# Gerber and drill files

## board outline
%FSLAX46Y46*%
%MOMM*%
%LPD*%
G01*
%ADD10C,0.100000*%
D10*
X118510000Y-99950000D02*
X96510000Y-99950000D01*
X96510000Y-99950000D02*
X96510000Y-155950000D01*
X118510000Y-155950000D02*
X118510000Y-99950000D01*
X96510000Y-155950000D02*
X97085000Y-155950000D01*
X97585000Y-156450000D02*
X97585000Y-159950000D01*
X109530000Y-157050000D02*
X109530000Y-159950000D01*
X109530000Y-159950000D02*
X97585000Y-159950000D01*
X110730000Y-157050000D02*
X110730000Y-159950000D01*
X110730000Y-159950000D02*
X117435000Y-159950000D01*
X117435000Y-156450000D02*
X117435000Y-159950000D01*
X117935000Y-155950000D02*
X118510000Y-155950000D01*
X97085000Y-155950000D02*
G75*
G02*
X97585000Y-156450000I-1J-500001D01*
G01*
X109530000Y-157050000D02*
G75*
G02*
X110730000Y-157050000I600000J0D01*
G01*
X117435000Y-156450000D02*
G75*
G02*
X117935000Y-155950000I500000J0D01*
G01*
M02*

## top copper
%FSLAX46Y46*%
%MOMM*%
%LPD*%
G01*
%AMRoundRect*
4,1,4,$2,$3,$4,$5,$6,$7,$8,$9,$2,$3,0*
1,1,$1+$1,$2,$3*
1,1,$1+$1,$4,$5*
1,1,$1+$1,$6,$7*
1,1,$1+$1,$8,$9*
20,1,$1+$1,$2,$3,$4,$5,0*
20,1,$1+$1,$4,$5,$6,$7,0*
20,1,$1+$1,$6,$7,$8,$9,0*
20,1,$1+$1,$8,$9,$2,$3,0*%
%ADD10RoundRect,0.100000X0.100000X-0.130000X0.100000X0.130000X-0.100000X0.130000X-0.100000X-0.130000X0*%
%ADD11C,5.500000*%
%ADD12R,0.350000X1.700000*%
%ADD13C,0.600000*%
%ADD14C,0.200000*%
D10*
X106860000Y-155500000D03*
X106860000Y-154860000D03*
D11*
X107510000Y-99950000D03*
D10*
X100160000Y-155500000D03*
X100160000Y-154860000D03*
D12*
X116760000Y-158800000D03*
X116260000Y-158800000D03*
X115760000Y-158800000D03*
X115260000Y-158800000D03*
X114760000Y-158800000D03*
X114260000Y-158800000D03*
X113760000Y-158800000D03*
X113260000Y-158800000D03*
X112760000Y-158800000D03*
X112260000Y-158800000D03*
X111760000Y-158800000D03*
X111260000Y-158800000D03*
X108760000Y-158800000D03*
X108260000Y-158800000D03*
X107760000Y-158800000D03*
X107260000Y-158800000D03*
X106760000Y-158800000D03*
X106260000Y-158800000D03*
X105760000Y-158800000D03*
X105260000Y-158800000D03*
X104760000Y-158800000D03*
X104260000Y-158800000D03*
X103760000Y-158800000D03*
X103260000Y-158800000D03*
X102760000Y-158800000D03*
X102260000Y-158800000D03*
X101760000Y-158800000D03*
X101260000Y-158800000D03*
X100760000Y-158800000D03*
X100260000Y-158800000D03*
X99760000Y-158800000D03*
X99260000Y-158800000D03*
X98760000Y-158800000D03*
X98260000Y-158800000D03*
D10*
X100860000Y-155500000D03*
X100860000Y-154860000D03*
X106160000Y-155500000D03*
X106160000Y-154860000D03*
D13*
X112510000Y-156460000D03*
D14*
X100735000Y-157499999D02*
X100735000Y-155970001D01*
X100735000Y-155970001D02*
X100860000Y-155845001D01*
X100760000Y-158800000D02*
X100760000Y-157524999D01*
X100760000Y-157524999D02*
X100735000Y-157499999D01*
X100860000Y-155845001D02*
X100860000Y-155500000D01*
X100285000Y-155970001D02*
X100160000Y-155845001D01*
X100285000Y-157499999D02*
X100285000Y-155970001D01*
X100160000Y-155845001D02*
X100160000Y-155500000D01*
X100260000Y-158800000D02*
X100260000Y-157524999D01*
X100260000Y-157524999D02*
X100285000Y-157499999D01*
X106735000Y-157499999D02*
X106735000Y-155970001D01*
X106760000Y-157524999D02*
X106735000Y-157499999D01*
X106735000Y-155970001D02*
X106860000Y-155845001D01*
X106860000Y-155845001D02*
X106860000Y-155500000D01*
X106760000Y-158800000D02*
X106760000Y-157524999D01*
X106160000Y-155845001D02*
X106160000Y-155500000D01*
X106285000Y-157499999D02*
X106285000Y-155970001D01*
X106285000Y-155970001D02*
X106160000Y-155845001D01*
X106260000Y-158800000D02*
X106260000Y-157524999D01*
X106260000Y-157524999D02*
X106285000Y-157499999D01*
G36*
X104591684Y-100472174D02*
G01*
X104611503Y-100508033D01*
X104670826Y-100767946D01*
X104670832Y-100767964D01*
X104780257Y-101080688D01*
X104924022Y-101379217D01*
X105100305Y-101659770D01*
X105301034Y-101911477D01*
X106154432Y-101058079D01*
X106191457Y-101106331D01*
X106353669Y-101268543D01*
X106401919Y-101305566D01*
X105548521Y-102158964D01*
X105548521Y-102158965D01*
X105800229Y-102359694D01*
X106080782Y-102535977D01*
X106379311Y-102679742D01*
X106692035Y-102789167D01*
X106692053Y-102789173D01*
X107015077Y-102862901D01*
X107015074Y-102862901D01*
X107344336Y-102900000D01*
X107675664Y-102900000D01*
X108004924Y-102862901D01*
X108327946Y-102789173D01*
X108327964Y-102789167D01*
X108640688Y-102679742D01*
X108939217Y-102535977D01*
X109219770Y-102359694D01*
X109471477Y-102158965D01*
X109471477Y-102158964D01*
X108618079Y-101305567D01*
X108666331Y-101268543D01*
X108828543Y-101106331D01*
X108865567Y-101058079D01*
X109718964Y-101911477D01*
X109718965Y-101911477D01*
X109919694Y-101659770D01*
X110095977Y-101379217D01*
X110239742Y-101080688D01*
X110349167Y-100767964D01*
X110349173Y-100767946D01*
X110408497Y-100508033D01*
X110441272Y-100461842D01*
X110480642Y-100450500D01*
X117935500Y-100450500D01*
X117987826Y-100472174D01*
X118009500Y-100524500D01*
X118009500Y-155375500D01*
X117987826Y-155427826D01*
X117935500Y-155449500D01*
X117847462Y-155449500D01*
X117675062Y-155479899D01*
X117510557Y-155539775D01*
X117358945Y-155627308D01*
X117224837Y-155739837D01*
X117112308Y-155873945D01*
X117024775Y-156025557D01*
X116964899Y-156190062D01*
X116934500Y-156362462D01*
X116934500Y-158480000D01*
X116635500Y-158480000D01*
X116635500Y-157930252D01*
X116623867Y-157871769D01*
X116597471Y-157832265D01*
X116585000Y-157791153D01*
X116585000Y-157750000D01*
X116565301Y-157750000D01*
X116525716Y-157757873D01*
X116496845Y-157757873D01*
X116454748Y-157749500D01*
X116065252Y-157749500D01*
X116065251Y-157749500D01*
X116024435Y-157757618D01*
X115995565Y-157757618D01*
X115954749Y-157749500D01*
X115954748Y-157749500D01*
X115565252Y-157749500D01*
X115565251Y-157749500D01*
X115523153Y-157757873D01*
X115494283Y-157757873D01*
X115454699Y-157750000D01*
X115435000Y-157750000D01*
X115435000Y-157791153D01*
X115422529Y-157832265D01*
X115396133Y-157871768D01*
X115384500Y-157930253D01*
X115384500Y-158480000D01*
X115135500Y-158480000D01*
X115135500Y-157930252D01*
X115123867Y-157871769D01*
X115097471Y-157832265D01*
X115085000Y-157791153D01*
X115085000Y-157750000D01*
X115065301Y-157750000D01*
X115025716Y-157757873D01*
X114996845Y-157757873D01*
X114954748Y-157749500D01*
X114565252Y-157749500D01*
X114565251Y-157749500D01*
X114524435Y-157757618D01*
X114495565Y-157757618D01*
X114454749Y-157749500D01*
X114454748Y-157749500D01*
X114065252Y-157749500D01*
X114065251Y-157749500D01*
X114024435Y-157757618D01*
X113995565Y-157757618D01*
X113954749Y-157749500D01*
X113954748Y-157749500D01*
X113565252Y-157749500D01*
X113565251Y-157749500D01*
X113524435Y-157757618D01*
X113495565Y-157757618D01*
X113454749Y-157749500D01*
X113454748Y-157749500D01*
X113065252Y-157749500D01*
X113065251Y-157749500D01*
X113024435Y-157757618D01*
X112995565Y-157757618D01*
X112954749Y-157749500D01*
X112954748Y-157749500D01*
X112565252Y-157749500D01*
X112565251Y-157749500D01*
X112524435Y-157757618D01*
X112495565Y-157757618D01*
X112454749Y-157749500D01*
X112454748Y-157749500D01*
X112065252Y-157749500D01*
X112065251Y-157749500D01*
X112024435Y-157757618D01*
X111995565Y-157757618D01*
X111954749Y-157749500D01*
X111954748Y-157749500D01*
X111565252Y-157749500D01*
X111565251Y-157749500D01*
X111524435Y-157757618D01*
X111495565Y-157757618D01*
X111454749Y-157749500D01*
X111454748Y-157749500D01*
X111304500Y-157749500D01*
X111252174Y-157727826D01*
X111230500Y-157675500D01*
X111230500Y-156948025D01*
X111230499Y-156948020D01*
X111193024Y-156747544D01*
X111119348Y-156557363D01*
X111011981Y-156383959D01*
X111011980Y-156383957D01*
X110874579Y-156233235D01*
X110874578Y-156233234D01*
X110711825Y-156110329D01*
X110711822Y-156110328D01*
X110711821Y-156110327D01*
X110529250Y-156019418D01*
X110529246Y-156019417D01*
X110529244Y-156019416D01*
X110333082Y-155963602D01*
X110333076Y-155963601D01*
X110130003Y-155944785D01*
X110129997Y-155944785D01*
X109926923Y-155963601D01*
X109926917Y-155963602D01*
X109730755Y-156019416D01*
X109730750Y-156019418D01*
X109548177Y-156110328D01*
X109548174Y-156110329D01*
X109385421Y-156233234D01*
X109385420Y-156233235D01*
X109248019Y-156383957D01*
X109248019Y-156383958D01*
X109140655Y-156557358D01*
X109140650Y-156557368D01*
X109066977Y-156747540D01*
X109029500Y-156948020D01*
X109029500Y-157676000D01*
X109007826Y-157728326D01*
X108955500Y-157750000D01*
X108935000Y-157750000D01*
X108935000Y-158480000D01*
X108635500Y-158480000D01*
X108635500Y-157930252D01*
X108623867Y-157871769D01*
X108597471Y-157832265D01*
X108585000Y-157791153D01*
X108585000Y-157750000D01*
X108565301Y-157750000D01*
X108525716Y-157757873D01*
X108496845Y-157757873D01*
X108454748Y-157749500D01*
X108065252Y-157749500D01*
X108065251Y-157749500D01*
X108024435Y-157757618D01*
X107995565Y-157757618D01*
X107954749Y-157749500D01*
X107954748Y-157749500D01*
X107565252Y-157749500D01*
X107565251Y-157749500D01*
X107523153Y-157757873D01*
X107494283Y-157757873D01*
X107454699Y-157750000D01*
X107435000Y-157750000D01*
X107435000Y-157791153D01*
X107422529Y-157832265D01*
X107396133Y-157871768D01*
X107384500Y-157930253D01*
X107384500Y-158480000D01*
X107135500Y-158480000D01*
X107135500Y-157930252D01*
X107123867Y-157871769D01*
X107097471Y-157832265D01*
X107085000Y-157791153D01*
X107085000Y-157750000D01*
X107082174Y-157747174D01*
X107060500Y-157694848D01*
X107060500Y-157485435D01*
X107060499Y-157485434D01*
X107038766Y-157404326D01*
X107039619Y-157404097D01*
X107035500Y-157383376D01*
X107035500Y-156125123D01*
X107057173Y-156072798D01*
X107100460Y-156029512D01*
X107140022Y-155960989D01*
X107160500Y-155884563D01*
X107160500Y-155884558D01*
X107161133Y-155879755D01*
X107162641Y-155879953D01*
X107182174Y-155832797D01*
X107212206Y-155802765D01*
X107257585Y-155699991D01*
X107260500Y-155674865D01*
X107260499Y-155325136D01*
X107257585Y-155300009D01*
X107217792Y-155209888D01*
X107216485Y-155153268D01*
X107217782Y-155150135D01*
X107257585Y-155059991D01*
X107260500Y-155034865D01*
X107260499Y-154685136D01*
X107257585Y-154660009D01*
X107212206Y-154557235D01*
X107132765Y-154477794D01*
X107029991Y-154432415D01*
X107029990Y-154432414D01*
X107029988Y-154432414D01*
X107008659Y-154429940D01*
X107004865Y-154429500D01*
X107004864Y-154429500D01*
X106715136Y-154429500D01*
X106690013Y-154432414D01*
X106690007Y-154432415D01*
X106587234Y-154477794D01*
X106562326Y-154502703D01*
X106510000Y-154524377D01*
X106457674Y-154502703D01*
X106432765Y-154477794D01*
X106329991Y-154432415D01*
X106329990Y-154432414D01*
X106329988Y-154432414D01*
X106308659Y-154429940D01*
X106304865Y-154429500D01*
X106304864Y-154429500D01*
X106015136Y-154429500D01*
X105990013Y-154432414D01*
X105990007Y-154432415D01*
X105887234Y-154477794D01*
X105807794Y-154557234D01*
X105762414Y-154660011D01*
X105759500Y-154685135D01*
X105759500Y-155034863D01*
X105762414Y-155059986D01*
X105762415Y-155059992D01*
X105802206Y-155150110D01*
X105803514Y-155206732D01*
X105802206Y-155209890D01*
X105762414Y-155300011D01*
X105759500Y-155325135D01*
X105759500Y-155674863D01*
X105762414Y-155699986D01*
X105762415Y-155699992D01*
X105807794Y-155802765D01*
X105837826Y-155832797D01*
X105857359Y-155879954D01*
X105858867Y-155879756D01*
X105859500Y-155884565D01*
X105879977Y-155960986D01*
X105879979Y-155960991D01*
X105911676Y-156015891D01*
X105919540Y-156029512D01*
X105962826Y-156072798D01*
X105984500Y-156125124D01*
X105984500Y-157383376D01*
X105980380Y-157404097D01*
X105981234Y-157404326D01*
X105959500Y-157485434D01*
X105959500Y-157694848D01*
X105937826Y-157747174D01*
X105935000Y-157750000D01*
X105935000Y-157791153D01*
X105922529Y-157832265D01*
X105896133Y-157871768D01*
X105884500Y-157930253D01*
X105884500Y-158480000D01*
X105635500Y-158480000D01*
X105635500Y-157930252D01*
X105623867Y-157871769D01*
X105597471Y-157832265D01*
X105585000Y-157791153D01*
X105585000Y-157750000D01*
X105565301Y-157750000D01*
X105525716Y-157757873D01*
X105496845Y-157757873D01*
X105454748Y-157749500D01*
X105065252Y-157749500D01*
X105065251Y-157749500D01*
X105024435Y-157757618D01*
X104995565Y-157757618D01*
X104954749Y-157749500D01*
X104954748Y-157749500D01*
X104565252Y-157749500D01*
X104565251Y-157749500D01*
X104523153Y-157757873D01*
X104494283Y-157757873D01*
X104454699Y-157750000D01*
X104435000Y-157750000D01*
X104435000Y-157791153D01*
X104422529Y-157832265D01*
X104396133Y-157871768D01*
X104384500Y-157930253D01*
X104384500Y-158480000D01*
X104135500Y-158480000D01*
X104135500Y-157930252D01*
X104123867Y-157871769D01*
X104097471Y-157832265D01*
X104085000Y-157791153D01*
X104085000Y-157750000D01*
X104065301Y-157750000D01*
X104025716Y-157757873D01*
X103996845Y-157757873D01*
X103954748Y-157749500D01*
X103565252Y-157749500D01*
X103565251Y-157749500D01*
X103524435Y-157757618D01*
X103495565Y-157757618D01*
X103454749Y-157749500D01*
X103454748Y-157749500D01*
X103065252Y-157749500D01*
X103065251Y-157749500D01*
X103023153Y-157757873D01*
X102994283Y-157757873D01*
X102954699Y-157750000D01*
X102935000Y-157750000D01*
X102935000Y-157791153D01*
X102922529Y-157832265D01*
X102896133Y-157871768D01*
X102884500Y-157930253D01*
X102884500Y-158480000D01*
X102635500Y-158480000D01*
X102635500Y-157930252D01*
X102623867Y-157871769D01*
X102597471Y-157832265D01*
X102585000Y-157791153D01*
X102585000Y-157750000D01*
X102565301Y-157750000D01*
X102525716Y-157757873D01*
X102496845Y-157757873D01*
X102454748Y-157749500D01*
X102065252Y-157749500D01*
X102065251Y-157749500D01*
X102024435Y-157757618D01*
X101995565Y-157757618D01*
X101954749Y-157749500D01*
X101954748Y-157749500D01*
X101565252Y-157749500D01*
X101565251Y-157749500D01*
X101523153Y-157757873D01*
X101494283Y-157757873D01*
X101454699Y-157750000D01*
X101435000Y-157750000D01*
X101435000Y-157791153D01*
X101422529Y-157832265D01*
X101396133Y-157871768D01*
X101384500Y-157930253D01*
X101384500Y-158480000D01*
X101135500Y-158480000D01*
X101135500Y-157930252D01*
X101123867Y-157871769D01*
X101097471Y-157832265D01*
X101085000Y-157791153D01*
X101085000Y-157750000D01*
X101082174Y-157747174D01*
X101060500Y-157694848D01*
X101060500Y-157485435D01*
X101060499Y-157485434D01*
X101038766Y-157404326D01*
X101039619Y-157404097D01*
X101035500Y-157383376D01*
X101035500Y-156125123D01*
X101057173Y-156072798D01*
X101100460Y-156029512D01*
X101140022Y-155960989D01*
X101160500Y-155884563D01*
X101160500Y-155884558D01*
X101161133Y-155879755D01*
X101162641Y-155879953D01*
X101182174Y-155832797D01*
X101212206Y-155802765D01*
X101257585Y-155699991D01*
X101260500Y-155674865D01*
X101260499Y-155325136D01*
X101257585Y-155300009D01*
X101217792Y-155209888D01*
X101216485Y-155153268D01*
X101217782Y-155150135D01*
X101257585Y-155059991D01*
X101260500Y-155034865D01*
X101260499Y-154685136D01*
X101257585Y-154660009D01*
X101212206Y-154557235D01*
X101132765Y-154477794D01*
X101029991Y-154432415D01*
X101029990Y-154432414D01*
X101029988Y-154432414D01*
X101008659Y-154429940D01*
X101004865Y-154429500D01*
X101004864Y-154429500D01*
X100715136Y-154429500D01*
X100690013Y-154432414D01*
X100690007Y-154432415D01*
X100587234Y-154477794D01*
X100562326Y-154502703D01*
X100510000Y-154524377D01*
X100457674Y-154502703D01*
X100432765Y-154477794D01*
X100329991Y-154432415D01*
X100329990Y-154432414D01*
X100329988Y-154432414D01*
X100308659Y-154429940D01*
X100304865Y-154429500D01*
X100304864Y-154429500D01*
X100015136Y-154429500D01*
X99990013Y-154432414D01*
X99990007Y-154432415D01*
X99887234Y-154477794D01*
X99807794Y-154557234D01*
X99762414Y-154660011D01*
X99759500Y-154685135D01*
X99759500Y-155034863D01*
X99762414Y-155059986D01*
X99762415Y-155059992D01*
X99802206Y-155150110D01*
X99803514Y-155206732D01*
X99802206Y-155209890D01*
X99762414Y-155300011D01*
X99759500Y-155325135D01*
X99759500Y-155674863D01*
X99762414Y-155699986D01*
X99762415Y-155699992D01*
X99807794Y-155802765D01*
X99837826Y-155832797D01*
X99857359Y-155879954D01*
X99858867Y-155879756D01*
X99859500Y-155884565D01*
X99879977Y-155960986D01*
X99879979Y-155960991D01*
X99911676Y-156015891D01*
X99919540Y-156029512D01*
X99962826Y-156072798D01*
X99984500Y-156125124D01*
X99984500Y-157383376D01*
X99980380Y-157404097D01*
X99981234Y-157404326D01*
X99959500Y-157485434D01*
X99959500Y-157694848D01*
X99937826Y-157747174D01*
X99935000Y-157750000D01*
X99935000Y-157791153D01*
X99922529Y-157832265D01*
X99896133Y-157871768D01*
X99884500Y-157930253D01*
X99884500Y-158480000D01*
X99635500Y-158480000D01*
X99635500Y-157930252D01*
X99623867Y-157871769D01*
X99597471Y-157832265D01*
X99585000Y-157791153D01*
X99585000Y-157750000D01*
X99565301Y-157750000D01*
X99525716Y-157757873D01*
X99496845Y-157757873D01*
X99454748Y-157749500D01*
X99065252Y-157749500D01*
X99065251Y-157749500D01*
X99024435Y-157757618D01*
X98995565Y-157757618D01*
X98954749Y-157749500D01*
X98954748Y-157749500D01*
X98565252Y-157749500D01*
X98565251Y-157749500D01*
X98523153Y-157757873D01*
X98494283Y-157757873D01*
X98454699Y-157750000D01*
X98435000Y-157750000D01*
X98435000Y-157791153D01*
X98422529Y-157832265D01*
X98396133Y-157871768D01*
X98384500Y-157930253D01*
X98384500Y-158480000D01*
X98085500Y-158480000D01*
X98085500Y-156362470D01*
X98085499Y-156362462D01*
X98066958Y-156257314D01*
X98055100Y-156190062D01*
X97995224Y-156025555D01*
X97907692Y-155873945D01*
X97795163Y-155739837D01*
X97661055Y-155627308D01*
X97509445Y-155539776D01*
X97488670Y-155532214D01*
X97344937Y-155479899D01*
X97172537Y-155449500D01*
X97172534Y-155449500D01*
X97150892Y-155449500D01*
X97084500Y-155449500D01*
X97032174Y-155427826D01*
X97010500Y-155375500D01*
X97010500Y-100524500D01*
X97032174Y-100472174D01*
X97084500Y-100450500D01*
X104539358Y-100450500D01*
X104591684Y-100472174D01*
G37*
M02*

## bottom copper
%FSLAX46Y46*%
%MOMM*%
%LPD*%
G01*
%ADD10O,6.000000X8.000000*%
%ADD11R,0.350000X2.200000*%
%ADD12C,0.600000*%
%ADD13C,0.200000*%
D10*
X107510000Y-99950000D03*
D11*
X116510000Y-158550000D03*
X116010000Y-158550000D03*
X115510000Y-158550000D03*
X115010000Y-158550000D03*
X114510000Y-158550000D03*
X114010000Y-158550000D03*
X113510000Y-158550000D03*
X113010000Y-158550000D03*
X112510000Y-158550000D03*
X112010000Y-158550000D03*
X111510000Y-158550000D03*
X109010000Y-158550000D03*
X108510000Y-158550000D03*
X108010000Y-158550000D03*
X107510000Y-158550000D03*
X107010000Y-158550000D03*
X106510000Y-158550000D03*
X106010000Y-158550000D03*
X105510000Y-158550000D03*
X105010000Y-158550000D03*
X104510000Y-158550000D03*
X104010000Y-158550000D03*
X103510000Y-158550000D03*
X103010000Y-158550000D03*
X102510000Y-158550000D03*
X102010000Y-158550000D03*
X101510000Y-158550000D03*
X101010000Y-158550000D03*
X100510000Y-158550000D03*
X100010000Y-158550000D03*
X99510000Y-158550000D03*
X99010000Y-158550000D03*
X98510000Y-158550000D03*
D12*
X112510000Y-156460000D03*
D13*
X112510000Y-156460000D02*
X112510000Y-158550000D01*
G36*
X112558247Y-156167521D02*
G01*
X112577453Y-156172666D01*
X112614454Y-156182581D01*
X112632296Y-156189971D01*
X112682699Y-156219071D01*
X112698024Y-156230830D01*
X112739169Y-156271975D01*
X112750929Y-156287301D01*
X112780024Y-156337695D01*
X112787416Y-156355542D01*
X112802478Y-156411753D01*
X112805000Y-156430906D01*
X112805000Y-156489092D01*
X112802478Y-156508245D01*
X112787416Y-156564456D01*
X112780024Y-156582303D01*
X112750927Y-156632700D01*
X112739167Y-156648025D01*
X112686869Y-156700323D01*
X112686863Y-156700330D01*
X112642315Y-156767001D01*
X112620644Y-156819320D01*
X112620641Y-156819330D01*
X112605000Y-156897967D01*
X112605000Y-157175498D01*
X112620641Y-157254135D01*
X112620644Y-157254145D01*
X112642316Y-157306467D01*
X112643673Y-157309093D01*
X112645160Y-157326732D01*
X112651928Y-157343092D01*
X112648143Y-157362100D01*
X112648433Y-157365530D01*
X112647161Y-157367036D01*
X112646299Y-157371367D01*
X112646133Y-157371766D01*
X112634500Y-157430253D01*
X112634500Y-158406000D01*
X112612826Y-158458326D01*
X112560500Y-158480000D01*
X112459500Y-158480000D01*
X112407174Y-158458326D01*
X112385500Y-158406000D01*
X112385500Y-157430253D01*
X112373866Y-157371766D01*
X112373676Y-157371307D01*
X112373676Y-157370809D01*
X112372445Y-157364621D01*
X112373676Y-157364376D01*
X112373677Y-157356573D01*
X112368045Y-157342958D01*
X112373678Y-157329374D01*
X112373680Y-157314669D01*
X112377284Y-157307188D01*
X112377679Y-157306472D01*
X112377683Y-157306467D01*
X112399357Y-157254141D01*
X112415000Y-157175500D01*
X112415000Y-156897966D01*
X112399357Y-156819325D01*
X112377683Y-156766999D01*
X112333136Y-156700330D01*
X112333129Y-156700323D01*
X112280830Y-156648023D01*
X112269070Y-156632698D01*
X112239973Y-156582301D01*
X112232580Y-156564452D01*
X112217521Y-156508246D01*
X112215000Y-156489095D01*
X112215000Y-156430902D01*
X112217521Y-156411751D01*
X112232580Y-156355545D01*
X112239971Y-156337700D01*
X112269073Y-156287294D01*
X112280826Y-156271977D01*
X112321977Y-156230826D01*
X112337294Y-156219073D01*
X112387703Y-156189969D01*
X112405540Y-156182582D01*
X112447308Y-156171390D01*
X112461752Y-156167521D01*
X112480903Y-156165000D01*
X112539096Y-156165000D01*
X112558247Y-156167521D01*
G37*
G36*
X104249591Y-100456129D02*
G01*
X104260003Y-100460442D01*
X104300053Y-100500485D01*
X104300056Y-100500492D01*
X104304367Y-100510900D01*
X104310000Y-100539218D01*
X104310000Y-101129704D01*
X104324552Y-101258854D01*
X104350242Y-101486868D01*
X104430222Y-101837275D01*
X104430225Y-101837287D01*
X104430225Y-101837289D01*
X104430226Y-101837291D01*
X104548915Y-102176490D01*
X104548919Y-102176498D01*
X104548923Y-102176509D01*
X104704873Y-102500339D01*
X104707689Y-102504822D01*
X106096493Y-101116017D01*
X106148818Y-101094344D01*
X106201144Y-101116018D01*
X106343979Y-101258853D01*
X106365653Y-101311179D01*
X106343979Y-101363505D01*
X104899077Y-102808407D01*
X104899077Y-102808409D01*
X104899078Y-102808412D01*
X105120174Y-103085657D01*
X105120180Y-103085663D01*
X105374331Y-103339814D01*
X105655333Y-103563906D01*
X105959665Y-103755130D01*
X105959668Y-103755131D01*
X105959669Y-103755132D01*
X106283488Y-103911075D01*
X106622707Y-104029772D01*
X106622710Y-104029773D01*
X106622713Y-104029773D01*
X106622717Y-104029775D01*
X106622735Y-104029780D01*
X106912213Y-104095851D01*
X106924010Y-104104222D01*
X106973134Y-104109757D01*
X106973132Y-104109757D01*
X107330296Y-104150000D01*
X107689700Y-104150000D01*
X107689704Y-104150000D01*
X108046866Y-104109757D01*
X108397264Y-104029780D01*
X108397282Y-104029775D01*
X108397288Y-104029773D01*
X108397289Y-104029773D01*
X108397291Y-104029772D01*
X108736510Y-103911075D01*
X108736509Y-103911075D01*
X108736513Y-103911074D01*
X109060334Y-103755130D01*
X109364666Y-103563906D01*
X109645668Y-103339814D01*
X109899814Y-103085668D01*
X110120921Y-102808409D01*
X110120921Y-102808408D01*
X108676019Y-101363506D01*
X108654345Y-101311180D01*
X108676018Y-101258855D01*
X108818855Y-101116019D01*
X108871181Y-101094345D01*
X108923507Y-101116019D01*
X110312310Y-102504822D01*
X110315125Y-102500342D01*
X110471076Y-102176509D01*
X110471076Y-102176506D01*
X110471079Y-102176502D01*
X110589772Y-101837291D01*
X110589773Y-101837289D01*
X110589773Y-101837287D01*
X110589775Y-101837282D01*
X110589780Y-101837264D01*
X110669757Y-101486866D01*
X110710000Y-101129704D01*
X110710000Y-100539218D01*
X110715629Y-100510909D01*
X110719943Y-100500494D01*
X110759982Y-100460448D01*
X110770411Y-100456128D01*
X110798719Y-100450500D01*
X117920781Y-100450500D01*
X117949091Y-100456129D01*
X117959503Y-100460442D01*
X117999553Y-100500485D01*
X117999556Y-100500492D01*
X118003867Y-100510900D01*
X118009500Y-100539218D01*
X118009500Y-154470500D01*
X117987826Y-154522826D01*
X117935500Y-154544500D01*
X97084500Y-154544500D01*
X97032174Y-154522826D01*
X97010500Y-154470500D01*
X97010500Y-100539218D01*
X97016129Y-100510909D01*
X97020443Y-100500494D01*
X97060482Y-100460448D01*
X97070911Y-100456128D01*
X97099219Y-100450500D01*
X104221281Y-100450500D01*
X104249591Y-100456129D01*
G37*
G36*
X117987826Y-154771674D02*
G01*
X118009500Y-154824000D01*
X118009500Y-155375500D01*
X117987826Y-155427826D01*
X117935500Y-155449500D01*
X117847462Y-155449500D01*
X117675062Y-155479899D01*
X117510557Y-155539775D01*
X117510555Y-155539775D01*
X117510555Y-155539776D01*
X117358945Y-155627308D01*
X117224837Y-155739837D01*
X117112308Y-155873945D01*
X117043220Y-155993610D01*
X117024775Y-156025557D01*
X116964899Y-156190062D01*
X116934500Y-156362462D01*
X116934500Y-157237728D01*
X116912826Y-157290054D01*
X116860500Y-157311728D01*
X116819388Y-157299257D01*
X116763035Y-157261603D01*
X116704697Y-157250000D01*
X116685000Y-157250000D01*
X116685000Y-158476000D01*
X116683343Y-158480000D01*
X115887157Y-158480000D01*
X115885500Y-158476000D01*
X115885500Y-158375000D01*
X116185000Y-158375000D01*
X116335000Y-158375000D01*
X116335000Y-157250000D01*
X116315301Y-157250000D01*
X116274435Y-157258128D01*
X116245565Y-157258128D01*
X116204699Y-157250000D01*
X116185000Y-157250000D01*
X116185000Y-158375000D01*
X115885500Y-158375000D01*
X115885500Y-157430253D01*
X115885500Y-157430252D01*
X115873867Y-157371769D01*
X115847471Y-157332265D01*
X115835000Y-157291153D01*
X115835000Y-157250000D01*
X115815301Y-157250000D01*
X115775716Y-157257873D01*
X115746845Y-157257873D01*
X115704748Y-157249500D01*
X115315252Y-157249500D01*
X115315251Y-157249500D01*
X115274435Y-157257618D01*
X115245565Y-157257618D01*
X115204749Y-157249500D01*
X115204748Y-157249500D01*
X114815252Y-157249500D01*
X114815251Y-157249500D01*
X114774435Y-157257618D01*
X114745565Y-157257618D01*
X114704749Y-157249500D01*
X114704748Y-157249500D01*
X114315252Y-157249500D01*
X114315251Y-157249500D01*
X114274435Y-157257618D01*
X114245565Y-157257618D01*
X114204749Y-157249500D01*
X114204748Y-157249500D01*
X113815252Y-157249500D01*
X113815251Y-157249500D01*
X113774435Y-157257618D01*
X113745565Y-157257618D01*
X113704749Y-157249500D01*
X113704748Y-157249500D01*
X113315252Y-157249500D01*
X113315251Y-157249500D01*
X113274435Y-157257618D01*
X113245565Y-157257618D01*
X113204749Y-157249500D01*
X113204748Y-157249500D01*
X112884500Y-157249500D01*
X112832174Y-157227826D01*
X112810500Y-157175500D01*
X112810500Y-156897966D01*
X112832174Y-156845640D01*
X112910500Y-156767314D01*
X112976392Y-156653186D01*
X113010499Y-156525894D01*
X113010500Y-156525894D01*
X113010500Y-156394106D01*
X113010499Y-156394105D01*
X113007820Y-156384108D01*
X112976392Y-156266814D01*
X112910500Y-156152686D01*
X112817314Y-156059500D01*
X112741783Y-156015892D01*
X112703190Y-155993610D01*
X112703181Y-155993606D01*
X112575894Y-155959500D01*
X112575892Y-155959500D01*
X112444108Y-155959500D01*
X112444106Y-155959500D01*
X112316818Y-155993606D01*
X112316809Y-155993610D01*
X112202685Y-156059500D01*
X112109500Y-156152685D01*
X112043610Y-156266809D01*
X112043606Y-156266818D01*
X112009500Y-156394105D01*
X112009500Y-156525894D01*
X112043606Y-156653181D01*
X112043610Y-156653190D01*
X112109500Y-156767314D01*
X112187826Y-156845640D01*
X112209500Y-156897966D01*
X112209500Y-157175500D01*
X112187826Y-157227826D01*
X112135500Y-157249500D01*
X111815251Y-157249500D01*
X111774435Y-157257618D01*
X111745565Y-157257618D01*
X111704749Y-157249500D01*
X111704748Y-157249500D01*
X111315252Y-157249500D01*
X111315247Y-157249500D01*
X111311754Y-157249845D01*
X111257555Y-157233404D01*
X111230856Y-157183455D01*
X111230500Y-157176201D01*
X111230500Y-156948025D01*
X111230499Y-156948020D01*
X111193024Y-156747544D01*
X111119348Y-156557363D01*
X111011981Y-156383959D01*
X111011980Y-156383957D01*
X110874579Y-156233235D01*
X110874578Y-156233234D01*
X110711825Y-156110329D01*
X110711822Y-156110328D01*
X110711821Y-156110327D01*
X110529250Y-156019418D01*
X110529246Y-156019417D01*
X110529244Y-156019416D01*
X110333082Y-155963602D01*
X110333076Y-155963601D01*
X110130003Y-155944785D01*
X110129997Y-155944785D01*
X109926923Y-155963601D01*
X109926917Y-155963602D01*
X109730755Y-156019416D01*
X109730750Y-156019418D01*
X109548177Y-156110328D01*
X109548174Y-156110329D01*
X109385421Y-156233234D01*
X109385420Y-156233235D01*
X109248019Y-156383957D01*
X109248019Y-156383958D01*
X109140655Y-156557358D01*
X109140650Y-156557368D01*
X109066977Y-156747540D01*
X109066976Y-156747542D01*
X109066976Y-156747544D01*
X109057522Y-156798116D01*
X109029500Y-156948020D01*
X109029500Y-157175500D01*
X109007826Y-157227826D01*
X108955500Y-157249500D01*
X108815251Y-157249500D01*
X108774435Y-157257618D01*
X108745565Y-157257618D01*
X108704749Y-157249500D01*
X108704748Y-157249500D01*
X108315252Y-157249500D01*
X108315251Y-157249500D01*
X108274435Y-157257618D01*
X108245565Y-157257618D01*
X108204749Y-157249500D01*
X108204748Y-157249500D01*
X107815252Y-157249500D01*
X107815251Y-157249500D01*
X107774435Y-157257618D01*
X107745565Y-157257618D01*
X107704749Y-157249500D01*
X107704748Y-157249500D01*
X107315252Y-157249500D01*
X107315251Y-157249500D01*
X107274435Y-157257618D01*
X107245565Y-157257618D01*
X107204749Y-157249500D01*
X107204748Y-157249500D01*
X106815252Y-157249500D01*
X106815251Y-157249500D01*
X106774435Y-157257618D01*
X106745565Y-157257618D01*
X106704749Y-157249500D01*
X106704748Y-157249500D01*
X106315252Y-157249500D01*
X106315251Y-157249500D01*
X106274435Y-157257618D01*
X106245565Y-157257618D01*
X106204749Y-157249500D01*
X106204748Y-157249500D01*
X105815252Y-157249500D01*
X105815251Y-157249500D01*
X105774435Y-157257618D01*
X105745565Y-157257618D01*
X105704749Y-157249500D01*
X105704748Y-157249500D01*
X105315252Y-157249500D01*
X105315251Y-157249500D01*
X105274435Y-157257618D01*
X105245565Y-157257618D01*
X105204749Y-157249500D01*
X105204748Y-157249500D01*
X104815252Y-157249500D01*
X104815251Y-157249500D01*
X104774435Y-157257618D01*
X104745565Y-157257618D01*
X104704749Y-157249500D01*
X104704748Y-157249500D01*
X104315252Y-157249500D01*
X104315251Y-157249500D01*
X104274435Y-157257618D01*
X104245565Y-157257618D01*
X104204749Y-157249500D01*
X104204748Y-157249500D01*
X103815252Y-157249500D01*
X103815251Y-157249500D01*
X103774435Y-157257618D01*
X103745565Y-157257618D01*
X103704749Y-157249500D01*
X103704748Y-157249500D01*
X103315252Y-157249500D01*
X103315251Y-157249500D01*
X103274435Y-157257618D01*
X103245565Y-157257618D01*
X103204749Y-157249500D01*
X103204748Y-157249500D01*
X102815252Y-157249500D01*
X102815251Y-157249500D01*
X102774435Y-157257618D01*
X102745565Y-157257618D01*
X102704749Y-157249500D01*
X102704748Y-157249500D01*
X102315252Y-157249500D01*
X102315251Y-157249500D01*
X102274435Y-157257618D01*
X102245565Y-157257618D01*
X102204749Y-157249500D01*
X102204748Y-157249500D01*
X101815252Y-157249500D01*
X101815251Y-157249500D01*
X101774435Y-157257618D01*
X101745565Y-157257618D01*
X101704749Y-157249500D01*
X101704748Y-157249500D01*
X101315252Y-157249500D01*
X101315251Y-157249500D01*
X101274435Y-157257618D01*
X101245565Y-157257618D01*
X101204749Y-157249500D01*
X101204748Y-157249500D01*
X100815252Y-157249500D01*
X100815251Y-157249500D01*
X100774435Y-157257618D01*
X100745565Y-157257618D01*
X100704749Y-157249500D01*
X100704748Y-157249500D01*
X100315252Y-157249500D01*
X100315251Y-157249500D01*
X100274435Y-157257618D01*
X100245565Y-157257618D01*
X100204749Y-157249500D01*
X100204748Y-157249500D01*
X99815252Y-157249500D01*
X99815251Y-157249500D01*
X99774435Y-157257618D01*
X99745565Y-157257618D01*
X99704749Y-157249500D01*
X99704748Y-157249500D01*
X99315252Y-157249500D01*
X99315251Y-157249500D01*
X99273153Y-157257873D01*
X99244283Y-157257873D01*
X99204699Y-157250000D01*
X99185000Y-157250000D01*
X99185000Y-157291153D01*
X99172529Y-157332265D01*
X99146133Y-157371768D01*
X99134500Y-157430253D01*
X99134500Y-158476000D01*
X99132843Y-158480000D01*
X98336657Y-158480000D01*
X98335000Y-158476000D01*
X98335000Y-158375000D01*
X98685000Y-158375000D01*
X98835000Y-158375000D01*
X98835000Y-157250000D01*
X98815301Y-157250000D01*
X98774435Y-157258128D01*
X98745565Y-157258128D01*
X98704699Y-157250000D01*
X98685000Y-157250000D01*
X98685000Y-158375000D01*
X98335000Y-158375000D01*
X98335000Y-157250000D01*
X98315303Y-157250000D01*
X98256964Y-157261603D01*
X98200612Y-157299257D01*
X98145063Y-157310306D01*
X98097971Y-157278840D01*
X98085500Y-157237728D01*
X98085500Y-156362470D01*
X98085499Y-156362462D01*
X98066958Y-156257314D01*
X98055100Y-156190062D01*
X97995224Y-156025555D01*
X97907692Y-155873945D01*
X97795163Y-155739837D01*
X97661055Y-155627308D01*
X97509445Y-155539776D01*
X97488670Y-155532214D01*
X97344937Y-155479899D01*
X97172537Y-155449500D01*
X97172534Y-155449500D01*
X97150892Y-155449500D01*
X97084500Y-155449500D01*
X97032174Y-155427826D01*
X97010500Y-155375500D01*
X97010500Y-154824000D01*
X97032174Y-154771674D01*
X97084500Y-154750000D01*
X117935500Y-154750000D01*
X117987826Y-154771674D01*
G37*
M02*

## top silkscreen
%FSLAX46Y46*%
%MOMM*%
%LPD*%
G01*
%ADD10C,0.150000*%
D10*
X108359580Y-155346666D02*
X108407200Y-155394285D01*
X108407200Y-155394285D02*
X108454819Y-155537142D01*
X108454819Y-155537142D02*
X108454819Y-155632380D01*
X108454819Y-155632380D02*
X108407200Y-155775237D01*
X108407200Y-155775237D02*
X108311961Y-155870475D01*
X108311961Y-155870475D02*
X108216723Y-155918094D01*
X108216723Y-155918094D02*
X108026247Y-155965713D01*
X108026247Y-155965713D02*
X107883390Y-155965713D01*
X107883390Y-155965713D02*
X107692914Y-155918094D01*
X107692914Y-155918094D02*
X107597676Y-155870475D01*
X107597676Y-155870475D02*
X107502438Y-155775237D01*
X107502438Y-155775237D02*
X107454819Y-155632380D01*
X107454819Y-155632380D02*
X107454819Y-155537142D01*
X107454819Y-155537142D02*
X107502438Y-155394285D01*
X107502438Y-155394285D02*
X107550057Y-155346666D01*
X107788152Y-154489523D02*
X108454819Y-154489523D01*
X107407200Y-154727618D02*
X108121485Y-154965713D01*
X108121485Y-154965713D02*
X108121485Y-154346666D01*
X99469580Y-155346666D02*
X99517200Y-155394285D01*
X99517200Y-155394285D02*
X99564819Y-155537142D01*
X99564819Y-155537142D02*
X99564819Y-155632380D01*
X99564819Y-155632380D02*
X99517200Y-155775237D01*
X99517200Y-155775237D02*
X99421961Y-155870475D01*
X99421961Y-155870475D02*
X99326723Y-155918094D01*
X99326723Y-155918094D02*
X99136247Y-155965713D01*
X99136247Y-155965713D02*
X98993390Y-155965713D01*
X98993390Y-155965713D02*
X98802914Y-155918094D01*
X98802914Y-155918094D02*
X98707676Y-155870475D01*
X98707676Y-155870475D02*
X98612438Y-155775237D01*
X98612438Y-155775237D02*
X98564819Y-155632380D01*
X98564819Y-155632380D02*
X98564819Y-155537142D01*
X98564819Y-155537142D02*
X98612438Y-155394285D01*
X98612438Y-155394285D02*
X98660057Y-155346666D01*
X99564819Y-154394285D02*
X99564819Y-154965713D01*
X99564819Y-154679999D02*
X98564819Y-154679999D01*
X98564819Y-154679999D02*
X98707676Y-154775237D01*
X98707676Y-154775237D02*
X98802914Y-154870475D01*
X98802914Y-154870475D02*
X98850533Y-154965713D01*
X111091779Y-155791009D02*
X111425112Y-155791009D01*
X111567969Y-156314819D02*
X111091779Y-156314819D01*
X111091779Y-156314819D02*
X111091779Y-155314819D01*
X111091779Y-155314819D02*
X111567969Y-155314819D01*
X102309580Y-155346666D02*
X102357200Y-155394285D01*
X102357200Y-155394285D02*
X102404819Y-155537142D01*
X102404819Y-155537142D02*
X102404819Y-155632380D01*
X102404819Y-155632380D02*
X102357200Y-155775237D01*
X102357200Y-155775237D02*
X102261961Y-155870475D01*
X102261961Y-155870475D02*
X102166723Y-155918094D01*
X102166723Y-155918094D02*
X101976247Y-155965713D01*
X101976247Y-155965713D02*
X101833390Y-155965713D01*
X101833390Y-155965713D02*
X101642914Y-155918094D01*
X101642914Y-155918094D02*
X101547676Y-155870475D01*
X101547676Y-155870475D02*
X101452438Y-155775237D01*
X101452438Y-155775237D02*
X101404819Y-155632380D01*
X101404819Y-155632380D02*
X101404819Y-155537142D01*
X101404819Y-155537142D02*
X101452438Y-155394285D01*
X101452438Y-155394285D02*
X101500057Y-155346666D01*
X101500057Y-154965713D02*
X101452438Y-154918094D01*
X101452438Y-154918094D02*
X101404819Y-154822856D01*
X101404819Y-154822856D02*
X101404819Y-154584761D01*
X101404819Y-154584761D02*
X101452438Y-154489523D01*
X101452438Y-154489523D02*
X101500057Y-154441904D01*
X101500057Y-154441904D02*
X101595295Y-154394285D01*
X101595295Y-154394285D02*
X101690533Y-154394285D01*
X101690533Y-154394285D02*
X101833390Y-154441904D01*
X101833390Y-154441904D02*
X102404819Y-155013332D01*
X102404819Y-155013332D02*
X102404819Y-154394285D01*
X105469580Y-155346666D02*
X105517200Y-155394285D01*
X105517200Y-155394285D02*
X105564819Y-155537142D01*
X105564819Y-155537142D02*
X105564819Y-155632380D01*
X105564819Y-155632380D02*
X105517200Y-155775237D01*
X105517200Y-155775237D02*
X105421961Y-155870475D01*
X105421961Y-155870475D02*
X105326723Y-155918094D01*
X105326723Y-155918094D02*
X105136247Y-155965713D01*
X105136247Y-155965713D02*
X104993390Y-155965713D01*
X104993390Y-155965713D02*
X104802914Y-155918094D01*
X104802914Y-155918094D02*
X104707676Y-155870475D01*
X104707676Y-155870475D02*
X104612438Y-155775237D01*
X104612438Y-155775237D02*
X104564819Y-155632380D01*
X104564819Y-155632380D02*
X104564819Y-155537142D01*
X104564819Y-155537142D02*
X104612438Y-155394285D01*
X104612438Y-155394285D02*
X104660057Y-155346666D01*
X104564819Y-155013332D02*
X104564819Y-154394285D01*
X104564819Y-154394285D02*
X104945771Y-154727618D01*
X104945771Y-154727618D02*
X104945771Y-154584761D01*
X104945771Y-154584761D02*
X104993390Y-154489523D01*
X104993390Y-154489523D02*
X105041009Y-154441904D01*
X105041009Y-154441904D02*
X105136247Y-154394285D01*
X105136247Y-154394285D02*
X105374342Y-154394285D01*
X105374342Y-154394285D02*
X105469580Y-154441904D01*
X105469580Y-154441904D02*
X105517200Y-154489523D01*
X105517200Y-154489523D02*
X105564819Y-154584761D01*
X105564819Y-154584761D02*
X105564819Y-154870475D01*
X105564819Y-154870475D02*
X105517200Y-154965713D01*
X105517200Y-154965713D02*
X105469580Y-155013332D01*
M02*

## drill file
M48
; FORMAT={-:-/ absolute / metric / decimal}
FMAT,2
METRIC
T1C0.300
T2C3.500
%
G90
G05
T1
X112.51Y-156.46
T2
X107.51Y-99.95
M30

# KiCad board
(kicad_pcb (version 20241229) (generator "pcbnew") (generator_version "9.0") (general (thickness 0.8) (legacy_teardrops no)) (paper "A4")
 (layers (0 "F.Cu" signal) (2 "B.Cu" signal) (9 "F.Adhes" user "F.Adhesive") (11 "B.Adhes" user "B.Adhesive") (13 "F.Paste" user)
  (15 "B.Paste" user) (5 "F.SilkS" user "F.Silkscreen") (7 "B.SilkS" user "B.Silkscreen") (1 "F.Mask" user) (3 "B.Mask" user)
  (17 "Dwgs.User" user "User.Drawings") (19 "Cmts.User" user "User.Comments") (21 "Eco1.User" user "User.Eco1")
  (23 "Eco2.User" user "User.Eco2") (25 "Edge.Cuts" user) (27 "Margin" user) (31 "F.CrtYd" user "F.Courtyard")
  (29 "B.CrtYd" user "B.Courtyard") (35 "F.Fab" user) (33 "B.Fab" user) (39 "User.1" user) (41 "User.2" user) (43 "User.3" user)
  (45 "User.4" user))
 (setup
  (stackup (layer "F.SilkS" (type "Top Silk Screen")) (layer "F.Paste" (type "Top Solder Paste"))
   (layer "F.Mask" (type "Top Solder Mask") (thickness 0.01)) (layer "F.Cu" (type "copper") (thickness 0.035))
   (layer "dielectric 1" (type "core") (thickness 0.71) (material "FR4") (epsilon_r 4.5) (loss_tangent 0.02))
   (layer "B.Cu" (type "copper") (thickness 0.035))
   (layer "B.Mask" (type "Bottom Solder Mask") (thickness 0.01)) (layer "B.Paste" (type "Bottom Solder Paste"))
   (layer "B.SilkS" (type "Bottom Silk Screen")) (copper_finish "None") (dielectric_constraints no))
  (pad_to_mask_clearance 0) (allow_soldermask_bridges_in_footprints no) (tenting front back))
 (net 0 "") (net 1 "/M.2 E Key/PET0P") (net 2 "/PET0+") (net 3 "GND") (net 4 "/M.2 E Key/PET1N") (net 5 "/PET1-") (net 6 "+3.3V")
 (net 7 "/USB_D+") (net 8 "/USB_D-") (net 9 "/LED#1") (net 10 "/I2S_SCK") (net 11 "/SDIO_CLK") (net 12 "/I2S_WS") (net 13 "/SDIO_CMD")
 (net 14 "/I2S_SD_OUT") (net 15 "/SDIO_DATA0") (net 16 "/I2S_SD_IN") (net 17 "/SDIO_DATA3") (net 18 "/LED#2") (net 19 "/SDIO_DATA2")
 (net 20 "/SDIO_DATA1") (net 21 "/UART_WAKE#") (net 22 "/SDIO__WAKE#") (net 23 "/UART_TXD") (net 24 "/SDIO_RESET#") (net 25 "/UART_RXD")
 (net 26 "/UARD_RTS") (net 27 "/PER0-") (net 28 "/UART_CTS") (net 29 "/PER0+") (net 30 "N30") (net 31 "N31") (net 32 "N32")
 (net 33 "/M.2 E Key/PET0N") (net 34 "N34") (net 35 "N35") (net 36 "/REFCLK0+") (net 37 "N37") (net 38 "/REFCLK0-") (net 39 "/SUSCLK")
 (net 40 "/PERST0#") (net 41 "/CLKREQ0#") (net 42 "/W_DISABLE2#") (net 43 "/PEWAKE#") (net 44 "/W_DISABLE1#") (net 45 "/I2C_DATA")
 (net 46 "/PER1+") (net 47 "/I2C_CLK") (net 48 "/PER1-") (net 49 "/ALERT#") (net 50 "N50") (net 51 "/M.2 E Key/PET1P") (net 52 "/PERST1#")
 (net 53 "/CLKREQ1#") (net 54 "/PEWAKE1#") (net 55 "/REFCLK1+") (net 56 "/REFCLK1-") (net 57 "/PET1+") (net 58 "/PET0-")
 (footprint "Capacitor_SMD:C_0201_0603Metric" (layer "F.Cu") (at 106.86 155.18 90)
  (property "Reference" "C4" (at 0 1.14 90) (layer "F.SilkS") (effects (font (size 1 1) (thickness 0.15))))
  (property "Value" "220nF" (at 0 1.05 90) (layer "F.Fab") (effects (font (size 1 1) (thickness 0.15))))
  (pad "" smd roundrect (at -0.345 0 90) (size 0.318 0.36) (layers "F.Paste") (roundrect_rratio 0.25))
  (pad "" smd roundrect (at 0.345 0 90) (size 0.318 0.36) (layers "F.Paste") (roundrect_rratio 0.25))
  (pad "1" smd roundrect (at -0.32 0 90) (size 0.46 0.4) (layers "F.Cu" "F.Mask") (roundrect_rratio 0.25) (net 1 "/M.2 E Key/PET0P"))
  (pad "2" smd roundrect (at 0.32 0 90) (size 0.46 0.4) (layers "F.Cu" "F.Mask") (roundrect_rratio 0.25) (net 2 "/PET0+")))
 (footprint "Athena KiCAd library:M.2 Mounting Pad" (layer "F.Cu") (at 107.51 99.95)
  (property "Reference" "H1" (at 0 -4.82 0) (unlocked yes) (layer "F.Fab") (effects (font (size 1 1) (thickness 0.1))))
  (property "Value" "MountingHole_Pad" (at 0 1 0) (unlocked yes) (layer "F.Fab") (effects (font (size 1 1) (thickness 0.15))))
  (pad "1" thru_hole circle (at 0 0) (size 5.5 5.5) (drill 3.5) (layers "*.Cu" "*.Mask") (remove_unused_layers no) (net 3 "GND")
   (padstack (mode front_inner_back)
    (layer "Inner" (shape circle) (size 5.5 5.5) (zone_connect -1))
    (layer "B.Cu" (shape oval) (size 6 8) (thermal_bridge_angle 45) (zone_connect -1)))))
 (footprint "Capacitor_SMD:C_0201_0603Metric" (layer "F.Cu") (at 100.16 155.18 90)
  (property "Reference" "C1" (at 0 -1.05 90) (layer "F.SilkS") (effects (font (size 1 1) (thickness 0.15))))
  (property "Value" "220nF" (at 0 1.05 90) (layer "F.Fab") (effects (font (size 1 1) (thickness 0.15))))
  (pad "" smd roundrect (at -0.345 0 90) (size 0.318 0.36) (layers "F.Paste") (roundrect_rratio 0.25))
  (pad "" smd roundrect (at 0.345 0 90) (size 0.318 0.36) (layers "F.Paste") (roundrect_rratio 0.25))
  (pad "1" smd roundrect (at -0.32 0 90) (size 0.46 0.4) (layers "F.Cu" "F.Mask") (roundrect_rratio 0.25) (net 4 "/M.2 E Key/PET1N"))
  (pad "2" smd roundrect (at 0.32 0 90) (size 0.46 0.4) (layers "F.Cu" "F.Mask") (roundrect_rratio 0.25) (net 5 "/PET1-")))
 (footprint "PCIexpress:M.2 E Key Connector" (layer "F.Cu") (at 107.51 158.84)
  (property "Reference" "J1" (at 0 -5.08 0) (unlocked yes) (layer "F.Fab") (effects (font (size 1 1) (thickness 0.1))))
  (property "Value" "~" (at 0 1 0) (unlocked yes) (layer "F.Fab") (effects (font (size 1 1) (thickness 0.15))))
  (fp_line (start -11 -2.89) (end -10.425 -2.89) (stroke (width 0.1) (type default)) (layer "Edge.Cuts"))
  (fp_line (start -9.925 -2.39) (end -9.925 1.11) (stroke (width 0.1) (type default)) (layer "Edge.Cuts"))
  (fp_line (start 2.02 -1.79) (end 2.02 1.11) (stroke (width 0.1) (type default)) (layer "Edge.Cuts"))
  (fp_line (start 2.02 1.11) (end -9.925 1.11) (stroke (width 0.1) (type default)) (layer "Edge.Cuts"))
  (fp_line (start 3.22 -1.79) (end 3.22 1.11) (stroke (width 0.1) (type default)) (layer "Edge.Cuts"))
  (fp_line (start 3.22 1.11) (end 9.925 1.11) (stroke (width 0.1) (type default)) (layer "Edge.Cuts"))
  (fp_line (start 9.925 -2.39) (end 9.925 1.11) (stroke (width 0.1) (type default)) (layer "Edge.Cuts"))
  (fp_line (start 10.425 -2.89) (end 11 -2.89) (stroke (width 0.1) (type default)) (layer "Edge.Cuts"))
  (fp_arc (start -10.425 -2.89) (mid -10.071447 -2.743553) (end -9.925 -2.39) (stroke (width 0.1) (type default)) (layer "Edge.Cuts"))
  (fp_arc (start 2.02 -1.79) (mid 2.62 -2.39) (end 3.22 -1.79) (stroke (width 0.1) (type default)) (layer "Edge.Cuts"))
  (fp_arc (start 9.925 -2.39) (mid 10.071447 -2.743553) (end 10.425 -2.89) (stroke (width 0.1) (type default)) (layer "Edge.Cuts"))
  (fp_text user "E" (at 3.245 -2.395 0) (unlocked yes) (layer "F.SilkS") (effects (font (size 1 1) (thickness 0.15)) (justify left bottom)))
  (pad "1" smd rect (at 9.25 -0.04 180) (size 0.35 1.7) (layers "F.Cu") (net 3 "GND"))
  (pad "2" smd rect (at 9 -0.29 180) (size 0.35 2.2) (layers "B.Cu") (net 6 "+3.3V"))
  (pad "3" smd rect (at 8.75 -0.04 180) (size 0.35 1.7) (layers "F.Cu") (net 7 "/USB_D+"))
  (pad "4" smd rect (at 8.5 -0.29 180) (size 0.35 2.2) (layers "B.Cu") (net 6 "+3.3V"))
  (pad "5" smd rect (at 8.25 -0.04 180) (size 0.35 1.7) (layers "F.Cu") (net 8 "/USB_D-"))
  (pad "6" smd rect (at 8 -0.29 180) (size 0.35 2.2) (layers "B.Cu") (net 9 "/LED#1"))
  (pad "7" smd rect (at 7.75 -0.04 180) (size 0.35 1.7) (layers "F.Cu") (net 3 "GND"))
  (pad "8" smd rect (at 7.5 -0.29 180) (size 0.35 2.2) (layers "B.Cu") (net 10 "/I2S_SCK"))
  (pad "9" smd rect (at 7.25 -0.04 180) (size 0.35 1.7) (layers "F.Cu") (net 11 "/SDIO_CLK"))
  (pad "10" smd rect (at 7 -0.29 180) (size 0.35 2.2) (layers "B.Cu") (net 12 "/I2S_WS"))
  (pad "11" smd rect (at 6.75 -0.04 180) (size 0.35 1.7) (layers "F.Cu") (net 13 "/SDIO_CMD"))
  (pad "12" smd rect (at 6.5 -0.29 180) (size 0.35 2.2) (layers "B.Cu") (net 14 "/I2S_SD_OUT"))
  (pad "13" smd rect (at 6.25 -0.04 180) (size 0.35 1.7) (layers "F.Cu") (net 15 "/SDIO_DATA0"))
  (pad "14" smd rect (at 6 -0.29 180) (size 0.35 2.2) (layers "B.Cu") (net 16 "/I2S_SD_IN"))
  (pad "15" smd rect (at 5.75 -0.04 180) (size 0.35 1.7) (layers "F.Cu") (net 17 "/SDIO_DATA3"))
  (pad "16" smd rect (at 5.5 -0.29 180) (size 0.35 2.2) (layers "B.Cu") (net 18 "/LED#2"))
  (pad "17" smd rect (at 5.25 -0.04 180) (size 0.35 1.7) (layers "F.Cu") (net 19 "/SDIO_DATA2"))
  (pad "18" smd rect (at 5 -0.29 180) (size 0.35 2.2) (layers "B.Cu") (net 3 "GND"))
  (pad "19" smd rect (at 4.75 -0.04 180) (size 0.35 1.7) (layers "F.Cu") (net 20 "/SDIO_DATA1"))
  (pad "20" smd rect (at 4.5 -0.29 180) (size 0.35 2.2) (layers "B.Cu") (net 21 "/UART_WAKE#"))
  (pad "21" smd rect (at 4.25 -0.04 180) (size 0.35 1.7) (layers "F.Cu") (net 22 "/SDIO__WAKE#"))
  (pad "22" smd rect (at 4 -0.29 180) (size 0.35 2.2) (layers "B.Cu") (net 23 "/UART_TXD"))
  (pad "23" smd rect (at 3.75 -0.04 180) (size 0.35 1.7) (layers "F.Cu") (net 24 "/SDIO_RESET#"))
  (pad "32" smd rect (at 1.5 -0.29 180) (size 0.35 2.2) (layers "B.Cu") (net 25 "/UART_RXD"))
  (pad "33" smd rect (at 1.25 -0.04 180) (size 0.35 1.7) (layers "F.Cu") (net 3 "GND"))
  (pad "34" smd rect (at 1 -0.29 180) (size 0.35 2.2) (layers "B.Cu") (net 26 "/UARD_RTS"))
  (pad "35" smd rect (at 0.75 -0.04 180) (size 0.35 1.7) (layers "F.Cu") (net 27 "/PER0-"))
  (pad "36" smd rect (at 0.5 -0.29 180) (size 0.35 2.2) (layers "B.Cu") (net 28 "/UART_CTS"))
  (pad "37" smd rect (at 0.25 -0.04 180) (size 0.35 1.7) (layers "F.Cu") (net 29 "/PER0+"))
  (pad "38" smd rect (at 0 -0.29 180) (size 0.35 2.2) (layers "B.Cu") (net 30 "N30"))
  (pad "39" smd rect (at -0.25 -0.04 180) (size 0.35 1.7) (layers "F.Cu") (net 3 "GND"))
  (pad "40" smd rect (at -0.5 -0.29 180) (size 0.35 2.2) (layers "B.Cu") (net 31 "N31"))
  (pad "41" smd rect (at -0.75 -0.04 180) (size 0.35 1.7) (layers "F.Cu") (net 1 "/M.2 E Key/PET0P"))
  (pad "42" smd rect (at -1 -0.29 180) (size 0.35 2.2) (layers "B.Cu") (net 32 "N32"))
  (pad "43" smd rect (at -1.25 -0.04 180) (size 0.35 1.7) (layers "F.Cu") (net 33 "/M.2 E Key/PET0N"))
  (pad "44" smd rect (at -1.5 -0.29 180) (size 0.35 2.2) (layers "B.Cu") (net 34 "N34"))
  (pad "45" smd rect (at -1.75 -0.04 180) (size 0.35 1.7) (layers "F.Cu") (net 3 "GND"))
  (pad "46" smd rect (at -2 -0.29 180) (size 0.35 2.2) (layers "B.Cu") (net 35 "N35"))
  (pad "47" smd rect (at -2.25 -0.04 180) (size 0.35 1.7) (layers "F.Cu") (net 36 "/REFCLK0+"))
  (pad "48" smd rect (at -2.5 -0.29 180) (size 0.35 2.2) (layers "B.Cu") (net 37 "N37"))
  (pad "49" smd rect (at -2.75 -0.04 180) (size 0.35 1.7) (layers "F.Cu") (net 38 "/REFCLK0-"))
  (pad "50" smd rect (at -3 -0.29 180) (size 0.35 2.2) (layers "B.Cu") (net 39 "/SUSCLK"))
  (pad "51" smd rect (at -3.25 -0.04 180) (size 0.35 1.7) (layers "F.Cu") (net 3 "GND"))
  (pad "52" smd rect (at -3.5 -0.29 180) (size 0.35 2.2) (layers "B.Cu") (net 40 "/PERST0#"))
  (pad "53" smd rect (at -3.75 -0.04 180) (size 0.35 1.7) (layers "F.Cu") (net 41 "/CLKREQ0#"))
  (pad "54" smd rect (at -4 -0.29 180) (size 0.35 2.2) (layers "B.Cu") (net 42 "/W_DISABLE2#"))
  (pad "55" smd rect (at -4.25 -0.04 180) (size 0.35 1.7) (layers "F.Cu") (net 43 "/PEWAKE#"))
  (pad "56" smd rect (at -4.5 -0.29 180) (size 0.35 2.2) (layers "B.Cu") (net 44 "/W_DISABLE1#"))
  (pad "57" smd rect (at -4.75 -0.04 180) (size 0.35 1.7) (layers "F.Cu") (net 3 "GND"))
  (pad "58" smd rect (at -5 -0.29 180) (size 0.35 2.2) (layers "B.Cu") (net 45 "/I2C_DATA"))
  (pad "59" smd rect (at -5.25 -0.04 180) (size 0.35 1.7) (layers "F.Cu") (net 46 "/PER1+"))
  (pad "60" smd rect (at -5.5 -0.29 180) (size 0.35 2.2) (layers "B.Cu") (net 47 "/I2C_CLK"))
  (pad "61" smd rect (at -5.75 -0.04 180) (size 0.35 1.7) (layers "F.Cu") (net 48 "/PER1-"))
  (pad "62" smd rect (at -6 -0.29 180) (size 0.35 2.2) (layers "B.Cu") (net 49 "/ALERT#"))
  (pad "63" smd rect (at -6.25 -0.04 180) (size 0.35 1.7) (layers "F.Cu") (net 3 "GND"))
  (pad "64" smd rect (at -6.5 -0.29 180) (size 0.35 2.2) (layers "B.Cu") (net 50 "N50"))
  (pad "65" smd rect (at -6.75 -0.04 180) (size 0.35 1.7) (layers "F.Cu") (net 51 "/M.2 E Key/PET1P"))
  (pad "66" smd rect (at -7 -0.29 180) (size 0.35 2.2) (layers "B.Cu") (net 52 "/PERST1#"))
  (pad "67" smd rect (at -7.25 -0.04 180) (size 0.35 1.7) (layers "F.Cu") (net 4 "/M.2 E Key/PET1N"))
  (pad "68" smd rect (at -7.5 -0.29 180) (size 0.35 2.2) (layers "B.Cu") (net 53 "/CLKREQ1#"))
  (pad "69" smd rect (at -7.75 -0.04 180) (size 0.35 1.7) (layers "F.Cu") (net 3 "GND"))
  (pad "70" smd rect (at -8 -0.29 180) (size 0.35 2.2) (layers "B.Cu") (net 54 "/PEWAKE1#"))
  (pad "71" smd rect (at -8.25 -0.04 180) (size 0.35 1.7) (layers "F.Cu") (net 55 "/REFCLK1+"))
  (pad "72" smd rect (at -8.5 -0.29 180) (size 0.35 2.2) (layers "B.Cu") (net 6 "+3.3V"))
  (pad "73" smd rect (at -8.75 -0.04 180) (size 0.35 1.7) (layers "F.Cu") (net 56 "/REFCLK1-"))
  (pad "74" smd rect (at -9 -0.29 180) (size 0.35 2.2) (layers "B.Cu") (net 6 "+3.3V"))
  (pad "75" smd rect (at -9.25 -0.04 180) (size 0.35 1.7) (layers "F.Cu") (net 3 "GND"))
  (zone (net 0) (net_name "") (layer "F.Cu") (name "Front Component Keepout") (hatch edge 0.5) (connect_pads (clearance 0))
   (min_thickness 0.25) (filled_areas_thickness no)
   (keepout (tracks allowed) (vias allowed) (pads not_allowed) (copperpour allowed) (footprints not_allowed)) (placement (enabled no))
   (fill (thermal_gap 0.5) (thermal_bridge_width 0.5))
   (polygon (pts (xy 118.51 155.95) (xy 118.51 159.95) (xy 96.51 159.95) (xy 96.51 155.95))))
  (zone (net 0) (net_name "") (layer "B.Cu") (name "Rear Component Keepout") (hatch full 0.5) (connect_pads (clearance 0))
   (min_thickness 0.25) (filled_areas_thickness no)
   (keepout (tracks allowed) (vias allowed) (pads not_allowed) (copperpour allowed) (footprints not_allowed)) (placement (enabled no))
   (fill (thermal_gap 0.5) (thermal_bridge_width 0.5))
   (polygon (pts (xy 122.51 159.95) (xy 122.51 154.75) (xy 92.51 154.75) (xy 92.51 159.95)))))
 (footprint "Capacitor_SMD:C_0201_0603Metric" (layer "F.Cu") (at 100.86 155.18 90)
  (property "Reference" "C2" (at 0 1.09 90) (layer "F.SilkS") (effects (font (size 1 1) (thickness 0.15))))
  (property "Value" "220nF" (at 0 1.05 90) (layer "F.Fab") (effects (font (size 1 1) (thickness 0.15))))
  (pad "" smd roundrect (at -0.345 0 90) (size 0.318 0.36) (layers "F.Paste") (roundrect_rratio 0.25))
  (pad "" smd roundrect (at 0.345 0 90) (size 0.318 0.36) (layers "F.Paste") (roundrect_rratio 0.25))
  (pad "1" smd roundrect (at -0.32 0 90) (size 0.46 0.4) (layers "F.Cu" "F.Mask") (roundrect_rratio 0.25) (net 51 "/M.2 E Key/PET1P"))
  (pad "2" smd roundrect (at 0.32 0 90) (size 0.46 0.4) (layers "F.Cu" "F.Mask") (roundrect_rratio 0.25) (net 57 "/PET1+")))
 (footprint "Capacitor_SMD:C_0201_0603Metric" (layer "F.Cu") (at 106.16 155.18 90)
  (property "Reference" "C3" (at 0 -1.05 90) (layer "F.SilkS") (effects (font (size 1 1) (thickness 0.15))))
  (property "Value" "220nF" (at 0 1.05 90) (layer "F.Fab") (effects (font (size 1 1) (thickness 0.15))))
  (pad "" smd roundrect (at -0.345 0 90) (size 0.318 0.36) (layers "F.Paste") (roundrect_rratio 0.25))
  (pad "" smd roundrect (at 0.345 0 90) (size 0.318 0.36) (layers "F.Paste") (roundrect_rratio 0.25))
  (pad "1" smd roundrect (at -0.32 0 90) (size 0.46 0.4) (layers "F.Cu" "F.Mask") (roundrect_rratio 0.25) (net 33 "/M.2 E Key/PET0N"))
  (pad "2" smd roundrect (at 0.32 0 90) (size 0.46 0.4) (layers "F.Cu" "F.Mask") (roundrect_rratio 0.25) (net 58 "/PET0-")))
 (gr_line (start 118.51 99.95) (end 96.51 99.95) (stroke (width 0.1) (type default)) (layer "Edge.Cuts"))
 (gr_line (start 96.51 99.95) (end 96.51 155.95) (stroke (width 0.1) (type default)) (layer "Edge.Cuts"))
 (gr_line (start 118.51 155.95) (end 118.51 99.95) (stroke (width 0.1) (type default)) (layer "Edge.Cuts"))
 (segment (start 100.735 157.499999) (end 100.735 155.970001) (width 0.2) (layer "F.Cu") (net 51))
 (segment (start 100.735 155.970001) (end 100.86 155.845001) (width 0.2) (layer "F.Cu") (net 51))
 (segment (start 100.76 158.8) (end 100.76 157.524999) (width 0.2) (layer "F.Cu") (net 51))
 (segment (start 100.76 157.524999) (end 100.735 157.499999) (width 0.2) (layer "F.Cu") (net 51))
 (segment (start 100.86 155.845001) (end 100.86 155.5) (width 0.2) (layer "F.Cu") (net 51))
 (segment (start 100.285 155.970001) (end 100.16 155.845001) (width 0.2) (layer "F.Cu") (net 4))
 (segment (start 100.285 157.499999) (end 100.285 155.970001) (width 0.2) (layer "F.Cu") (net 4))
 (segment (start 100.16 155.845001) (end 100.16 155.5) (width 0.2) (layer "F.Cu") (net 4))
 (segment (start 100.26 158.8) (end 100.26 157.524999) (width 0.2) (layer "F.Cu") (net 4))
 (segment (start 100.26 157.524999) (end 100.285 157.499999) (width 0.2) (layer "F.Cu") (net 4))
 (segment (start 106.735 157.499999) (end 106.735 155.970001) (width 0.2) (layer "F.Cu") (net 1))
 (segment (start 106.76 157.524999) (end 106.735 157.499999) (width 0.2) (layer "F.Cu") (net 1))
 (segment (start 106.735 155.970001) (end 106.86 155.845001) (width 0.2) (layer "F.Cu") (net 1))
 (segment (start 106.86 155.845001) (end 106.86 155.5) (width 0.2) (layer "F.Cu") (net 1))
 (segment (start 106.76 158.8) (end 106.76 157.524999) (width 0.2) (layer "F.Cu") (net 1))
 (segment (start 106.16 155.845001) (end 106.16 155.5) (width 0.2) (layer "F.Cu") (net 33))
 (segment (start 106.285 157.499999) (end 106.285 155.970001) (width 0.2) (layer "F.Cu") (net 33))
 (segment (start 106.285 155.970001) (end 106.16 155.845001) (width 0.2) (layer "F.Cu") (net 33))
 (segment (start 106.26 158.8) (end 106.26 157.524999) (width 0.2) (layer "F.Cu") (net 33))
 (segment (start 106.26 157.524999) (end 106.285 157.499999) (width 0.2) (layer "F.Cu") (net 33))
 (via (at 112.51 156.46) (size 0.6) (drill 0.3) (layers "F.Cu" "B.Cu") (free yes) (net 3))
 (segment (start 112.51 156.46) (end 112.51 158.55) (width 0.2) (layer "B.Cu") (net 3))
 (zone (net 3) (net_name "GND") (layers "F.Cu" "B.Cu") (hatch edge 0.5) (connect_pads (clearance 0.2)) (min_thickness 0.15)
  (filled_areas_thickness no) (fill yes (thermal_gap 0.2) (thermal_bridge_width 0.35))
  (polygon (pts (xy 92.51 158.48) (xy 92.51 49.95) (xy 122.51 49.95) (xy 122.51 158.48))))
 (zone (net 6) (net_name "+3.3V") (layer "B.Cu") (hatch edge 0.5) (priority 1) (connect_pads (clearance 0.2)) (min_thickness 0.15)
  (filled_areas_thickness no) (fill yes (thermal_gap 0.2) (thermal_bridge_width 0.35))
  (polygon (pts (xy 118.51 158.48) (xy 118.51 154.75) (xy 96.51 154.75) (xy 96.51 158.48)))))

